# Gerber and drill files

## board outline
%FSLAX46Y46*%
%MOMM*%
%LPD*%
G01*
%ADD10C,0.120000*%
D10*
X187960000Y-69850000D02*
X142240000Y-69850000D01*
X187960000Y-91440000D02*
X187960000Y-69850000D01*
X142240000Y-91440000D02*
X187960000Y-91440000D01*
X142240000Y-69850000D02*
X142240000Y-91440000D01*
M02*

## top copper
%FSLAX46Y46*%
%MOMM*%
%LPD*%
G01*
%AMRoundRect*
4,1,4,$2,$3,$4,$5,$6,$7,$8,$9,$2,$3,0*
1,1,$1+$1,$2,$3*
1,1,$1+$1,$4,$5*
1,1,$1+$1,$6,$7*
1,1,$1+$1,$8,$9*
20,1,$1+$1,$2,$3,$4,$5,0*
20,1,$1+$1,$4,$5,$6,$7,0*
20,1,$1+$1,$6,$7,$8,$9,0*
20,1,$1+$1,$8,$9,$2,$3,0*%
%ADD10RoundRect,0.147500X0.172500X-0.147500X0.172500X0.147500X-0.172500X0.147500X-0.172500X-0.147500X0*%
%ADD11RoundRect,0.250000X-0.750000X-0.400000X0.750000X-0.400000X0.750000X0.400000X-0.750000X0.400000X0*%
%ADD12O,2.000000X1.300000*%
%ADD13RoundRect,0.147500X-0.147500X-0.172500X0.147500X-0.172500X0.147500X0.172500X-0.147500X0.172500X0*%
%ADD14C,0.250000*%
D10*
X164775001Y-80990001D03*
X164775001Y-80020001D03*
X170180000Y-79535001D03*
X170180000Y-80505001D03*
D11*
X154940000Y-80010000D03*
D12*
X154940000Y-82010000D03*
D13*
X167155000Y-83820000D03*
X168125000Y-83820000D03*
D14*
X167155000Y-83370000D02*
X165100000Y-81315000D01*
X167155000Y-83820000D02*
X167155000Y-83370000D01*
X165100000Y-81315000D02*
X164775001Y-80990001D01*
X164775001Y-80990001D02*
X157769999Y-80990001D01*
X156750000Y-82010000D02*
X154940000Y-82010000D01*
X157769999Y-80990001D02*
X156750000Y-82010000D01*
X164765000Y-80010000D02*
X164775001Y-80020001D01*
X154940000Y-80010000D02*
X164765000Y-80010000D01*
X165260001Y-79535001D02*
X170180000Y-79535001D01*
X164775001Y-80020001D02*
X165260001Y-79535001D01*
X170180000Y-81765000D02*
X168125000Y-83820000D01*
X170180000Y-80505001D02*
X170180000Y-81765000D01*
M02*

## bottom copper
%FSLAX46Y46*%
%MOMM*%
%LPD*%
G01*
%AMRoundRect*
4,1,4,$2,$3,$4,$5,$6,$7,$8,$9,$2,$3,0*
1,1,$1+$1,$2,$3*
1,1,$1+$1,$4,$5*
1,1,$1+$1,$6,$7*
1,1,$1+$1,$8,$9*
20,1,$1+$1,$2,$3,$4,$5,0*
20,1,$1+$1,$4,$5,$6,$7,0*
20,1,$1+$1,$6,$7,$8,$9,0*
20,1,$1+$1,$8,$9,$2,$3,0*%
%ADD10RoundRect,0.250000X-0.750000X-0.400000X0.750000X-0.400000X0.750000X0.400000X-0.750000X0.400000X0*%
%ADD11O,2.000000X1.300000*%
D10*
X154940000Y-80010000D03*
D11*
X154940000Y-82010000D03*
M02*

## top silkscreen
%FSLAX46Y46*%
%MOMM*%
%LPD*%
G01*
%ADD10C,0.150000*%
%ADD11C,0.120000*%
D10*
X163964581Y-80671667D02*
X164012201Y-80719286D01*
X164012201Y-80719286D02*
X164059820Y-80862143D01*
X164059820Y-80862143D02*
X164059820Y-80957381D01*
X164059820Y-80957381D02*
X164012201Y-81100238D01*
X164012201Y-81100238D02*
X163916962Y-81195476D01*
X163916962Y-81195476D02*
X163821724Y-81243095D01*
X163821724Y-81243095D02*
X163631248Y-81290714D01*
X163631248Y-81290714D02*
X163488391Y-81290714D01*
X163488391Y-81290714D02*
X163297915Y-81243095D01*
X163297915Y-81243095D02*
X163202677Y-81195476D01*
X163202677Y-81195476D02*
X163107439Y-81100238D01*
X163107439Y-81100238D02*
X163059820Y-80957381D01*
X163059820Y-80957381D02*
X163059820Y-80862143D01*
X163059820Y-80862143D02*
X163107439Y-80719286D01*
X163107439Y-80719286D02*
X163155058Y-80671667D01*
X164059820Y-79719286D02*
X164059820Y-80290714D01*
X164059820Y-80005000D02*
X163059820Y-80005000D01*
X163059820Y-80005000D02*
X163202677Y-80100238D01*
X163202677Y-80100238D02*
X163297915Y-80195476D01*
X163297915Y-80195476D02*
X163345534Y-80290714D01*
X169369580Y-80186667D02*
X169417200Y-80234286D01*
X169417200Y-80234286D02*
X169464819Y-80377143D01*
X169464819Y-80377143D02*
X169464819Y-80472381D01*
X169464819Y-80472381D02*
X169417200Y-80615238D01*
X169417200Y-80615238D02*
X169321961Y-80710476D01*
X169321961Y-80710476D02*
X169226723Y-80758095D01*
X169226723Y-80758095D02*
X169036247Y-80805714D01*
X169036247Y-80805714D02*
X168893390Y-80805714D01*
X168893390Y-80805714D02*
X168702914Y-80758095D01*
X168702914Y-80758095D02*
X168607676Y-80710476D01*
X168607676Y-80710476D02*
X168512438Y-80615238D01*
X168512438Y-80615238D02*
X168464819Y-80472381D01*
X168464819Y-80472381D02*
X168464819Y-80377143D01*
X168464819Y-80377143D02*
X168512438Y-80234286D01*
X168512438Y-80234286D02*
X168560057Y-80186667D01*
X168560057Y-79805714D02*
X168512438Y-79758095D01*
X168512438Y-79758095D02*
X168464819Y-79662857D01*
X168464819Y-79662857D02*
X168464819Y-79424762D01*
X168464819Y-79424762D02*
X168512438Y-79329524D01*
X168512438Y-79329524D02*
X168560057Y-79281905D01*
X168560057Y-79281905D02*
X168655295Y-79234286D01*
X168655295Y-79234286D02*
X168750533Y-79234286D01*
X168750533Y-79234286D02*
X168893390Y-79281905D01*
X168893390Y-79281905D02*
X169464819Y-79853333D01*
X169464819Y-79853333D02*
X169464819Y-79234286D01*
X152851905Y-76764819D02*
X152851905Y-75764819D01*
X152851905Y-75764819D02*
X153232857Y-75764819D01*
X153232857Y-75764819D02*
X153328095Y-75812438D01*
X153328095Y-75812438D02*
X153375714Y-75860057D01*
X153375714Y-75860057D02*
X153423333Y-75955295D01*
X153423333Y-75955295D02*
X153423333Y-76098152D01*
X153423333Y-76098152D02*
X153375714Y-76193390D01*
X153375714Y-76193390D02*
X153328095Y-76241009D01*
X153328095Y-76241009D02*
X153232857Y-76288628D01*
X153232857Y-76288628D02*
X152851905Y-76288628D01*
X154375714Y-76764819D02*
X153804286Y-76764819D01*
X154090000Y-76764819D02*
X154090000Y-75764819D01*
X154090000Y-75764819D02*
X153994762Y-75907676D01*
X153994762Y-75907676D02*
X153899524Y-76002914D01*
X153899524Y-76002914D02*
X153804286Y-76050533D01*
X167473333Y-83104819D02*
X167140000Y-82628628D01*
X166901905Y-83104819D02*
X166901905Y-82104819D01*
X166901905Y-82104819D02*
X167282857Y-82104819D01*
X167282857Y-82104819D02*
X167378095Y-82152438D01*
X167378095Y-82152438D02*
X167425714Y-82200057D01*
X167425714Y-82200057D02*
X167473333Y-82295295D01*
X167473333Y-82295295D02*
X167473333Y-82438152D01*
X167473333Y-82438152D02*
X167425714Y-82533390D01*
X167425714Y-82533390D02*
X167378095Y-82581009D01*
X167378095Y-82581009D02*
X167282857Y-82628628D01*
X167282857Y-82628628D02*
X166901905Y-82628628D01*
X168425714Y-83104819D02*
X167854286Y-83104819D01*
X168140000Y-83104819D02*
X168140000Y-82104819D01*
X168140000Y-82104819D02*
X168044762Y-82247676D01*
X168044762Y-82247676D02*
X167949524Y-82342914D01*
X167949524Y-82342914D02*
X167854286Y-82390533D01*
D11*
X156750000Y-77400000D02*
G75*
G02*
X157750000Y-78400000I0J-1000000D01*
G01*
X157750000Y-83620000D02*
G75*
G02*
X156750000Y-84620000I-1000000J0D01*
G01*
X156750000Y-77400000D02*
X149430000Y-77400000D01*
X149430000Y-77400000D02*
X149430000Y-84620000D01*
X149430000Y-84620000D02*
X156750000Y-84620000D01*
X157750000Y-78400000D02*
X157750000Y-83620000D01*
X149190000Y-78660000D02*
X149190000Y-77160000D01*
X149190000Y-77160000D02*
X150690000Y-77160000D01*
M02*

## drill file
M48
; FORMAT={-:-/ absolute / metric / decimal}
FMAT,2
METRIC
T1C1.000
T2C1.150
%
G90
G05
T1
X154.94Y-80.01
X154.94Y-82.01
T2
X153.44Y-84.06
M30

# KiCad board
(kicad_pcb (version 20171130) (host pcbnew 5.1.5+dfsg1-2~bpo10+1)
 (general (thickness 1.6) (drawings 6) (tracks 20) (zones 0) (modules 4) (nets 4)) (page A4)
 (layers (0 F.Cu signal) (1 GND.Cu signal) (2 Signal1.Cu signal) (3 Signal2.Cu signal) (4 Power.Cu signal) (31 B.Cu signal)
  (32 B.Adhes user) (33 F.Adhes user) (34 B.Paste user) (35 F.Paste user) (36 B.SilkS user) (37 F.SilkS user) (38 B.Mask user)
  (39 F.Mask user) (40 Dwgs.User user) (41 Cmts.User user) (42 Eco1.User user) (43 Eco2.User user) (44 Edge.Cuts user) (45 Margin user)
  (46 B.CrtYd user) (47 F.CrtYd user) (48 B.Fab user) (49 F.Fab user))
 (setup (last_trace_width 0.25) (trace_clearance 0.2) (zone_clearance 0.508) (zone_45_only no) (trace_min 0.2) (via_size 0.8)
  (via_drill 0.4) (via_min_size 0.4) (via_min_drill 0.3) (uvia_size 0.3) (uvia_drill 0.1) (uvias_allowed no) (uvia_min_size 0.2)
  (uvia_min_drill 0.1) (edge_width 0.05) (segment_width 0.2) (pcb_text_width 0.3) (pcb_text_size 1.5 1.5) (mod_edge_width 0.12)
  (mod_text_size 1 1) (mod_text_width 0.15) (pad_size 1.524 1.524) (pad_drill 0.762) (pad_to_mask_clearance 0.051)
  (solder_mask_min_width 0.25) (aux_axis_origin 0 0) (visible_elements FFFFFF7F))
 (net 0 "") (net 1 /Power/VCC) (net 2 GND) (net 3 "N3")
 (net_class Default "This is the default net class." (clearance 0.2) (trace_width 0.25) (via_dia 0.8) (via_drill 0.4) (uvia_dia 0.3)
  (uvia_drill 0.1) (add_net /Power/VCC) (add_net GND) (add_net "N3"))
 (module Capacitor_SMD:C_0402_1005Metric (layer F.Cu) (at 164.775001 80.505001 90)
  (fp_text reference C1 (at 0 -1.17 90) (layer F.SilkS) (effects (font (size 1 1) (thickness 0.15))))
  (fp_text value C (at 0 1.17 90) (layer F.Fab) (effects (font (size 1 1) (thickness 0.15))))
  (pad 1 smd roundrect (at -0.485 0 90) (size 0.59 0.64) (layers F.Cu F.Paste F.Mask) (roundrect_rratio 0.25) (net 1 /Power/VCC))
  (pad 2 smd roundrect (at 0.485 0 90) (size 0.59 0.64) (layers F.Cu F.Paste F.Mask) (roundrect_rratio 0.25) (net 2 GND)))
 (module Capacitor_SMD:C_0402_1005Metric (layer F.Cu) (at 170.18 80.020001 90)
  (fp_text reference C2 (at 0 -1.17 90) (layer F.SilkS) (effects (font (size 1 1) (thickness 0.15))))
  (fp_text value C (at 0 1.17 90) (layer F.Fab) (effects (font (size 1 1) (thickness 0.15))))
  (pad 2 smd roundrect (at 0.485 0 90) (size 0.59 0.64) (layers F.Cu F.Paste F.Mask) (roundrect_rratio 0.25) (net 2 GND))
  (pad 1 smd roundrect (at -0.485 0 90) (size 0.59 0.64) (layers F.Cu F.Paste F.Mask) (roundrect_rratio 0.25) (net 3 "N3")))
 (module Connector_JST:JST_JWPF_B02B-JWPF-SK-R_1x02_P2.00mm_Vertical (layer F.Cu) (at 154.94 80.01)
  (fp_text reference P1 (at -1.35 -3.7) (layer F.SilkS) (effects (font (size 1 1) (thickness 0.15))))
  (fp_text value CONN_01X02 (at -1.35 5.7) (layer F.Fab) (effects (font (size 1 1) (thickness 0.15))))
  (fp_arc (start 1.81 -1.61) (end 1.81 -2.61) (angle 90) (layer F.SilkS) (width 0.12))
  (fp_arc (start 1.81 3.61) (end 2.81 3.61) (angle 90) (layer F.SilkS) (width 0.12))
  (fp_line (start 1.81 -2.61) (end -5.51 -2.61) (layer F.SilkS) (width 0.12))
  (fp_line (start -5.51 -2.61) (end -5.51 4.61) (layer F.SilkS) (width 0.12))
  (fp_line (start -5.51 4.61) (end 1.81 4.61) (layer F.SilkS) (width 0.12))
  (fp_line (start 2.81 -1.61) (end 2.81 3.61) (layer F.SilkS) (width 0.12))
  (fp_line (start -5.75 -1.35) (end -5.75 -2.85) (layer F.SilkS) (width 0.12))
  (fp_line (start -5.75 -2.85) (end -4.25 -2.85) (layer F.SilkS) (width 0.12))
  (pad 1 thru_hole roundrect (at 0 0) (size 2 1.3) (drill 1) (layers *.Cu *.Mask) (roundrect_rratio 0.192308) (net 2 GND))
  (pad 2 thru_hole oval (at 0 2) (size 2 1.3) (drill 1) (layers *.Cu *.Mask) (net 1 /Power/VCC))
  (pad "" np_thru_hole circle (at -1.5 4.05) (size 1.15 1.15) (drill 1.15) (layers *.Cu *.Mask)))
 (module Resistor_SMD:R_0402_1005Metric (layer F.Cu) (at 167.64 83.82)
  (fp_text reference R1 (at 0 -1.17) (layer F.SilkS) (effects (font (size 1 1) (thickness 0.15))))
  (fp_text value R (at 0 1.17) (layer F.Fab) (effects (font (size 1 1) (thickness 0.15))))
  (pad 1 smd roundrect (at -0.485 0) (size 0.59 0.64) (layers F.Cu F.Paste F.Mask) (roundrect_rratio 0.25) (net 1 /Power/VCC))
  (pad 2 smd roundrect (at 0.485 0) (size 0.59 0.64) (layers F.Cu F.Paste F.Mask) (roundrect_rratio 0.25) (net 3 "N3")))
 (gr_line (start 187.96 69.85) (end 142.24 69.85) (layer Edge.Cuts) (width 0.12))
 (gr_line (start 187.96 91.44) (end 187.96 69.85) (layer Edge.Cuts) (width 0.12))
 (gr_line (start 142.24 91.44) (end 187.96 91.44) (layer Edge.Cuts) (width 0.12))
 (gr_line (start 142.24 69.85) (end 142.24 91.44) (layer Edge.Cuts) (width 0.12))
 (segment (start 160 73) (end 180 73) (width 0.25) (layer GND.Cu) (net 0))
 (segment (start 180 73) (end 180 88) (width 0.25) (layer GND.Cu) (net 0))
 (segment (start 180 88) (end 160 88) (width 0.25) (layer Signal1.Cu) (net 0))
 (segment (start 160 88) (end 160 73) (width 0.25) (layer Signal1.Cu) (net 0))
 (segment (start 161 87) (end 179 87) (width 0.25) (layer Signal2.Cu) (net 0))
 (segment (start 179 87) (end 179 74) (width 0.25) (layer Signal2.Cu) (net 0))
 (segment (start 161 74) (end 179 74) (width 0.25) (layer Power.Cu) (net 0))
 (segment (start 161 74) (end 161 87) (width 0.25) (layer Power.Cu) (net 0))
 (segment (start 167.155 83.37) (end 165.1 81.315) (width 0.25) (layer F.Cu) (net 1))
 (segment (start 167.155 83.82) (end 167.155 83.37) (width 0.25) (layer F.Cu) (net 1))
 (segment (start 165.1 81.315) (end 164.775001 80.990001) (width 0.25) (layer F.Cu) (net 1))
 (segment (start 164.775001 80.990001) (end 157.769999 80.990001) (width 0.25) (layer F.Cu) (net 1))
 (segment (start 156.75 82.01) (end 154.94 82.01) (width 0.25) (layer F.Cu) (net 1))
 (segment (start 157.769999 80.990001) (end 156.75 82.01) (width 0.25) (layer F.Cu) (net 1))
 (segment (start 164.765 80.01) (end 164.775001 80.020001) (width 0.25) (layer F.Cu) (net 2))
 (segment (start 154.94 80.01) (end 164.765 80.01) (width 0.25) (layer F.Cu) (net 2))
 (segment (start 165.260001 79.535001) (end 170.18 79.535001) (width 0.25) (layer F.Cu) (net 2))
 (segment (start 164.775001 80.020001) (end 165.260001 79.535001) (width 0.25) (layer F.Cu) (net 2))
 (segment (start 170.18 81.765) (end 168.125 83.82) (width 0.25) (layer F.Cu) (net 3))
 (segment (start 170.18 80.505001) (end 170.18 81.765) (width 0.25) (layer F.Cu) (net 3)))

